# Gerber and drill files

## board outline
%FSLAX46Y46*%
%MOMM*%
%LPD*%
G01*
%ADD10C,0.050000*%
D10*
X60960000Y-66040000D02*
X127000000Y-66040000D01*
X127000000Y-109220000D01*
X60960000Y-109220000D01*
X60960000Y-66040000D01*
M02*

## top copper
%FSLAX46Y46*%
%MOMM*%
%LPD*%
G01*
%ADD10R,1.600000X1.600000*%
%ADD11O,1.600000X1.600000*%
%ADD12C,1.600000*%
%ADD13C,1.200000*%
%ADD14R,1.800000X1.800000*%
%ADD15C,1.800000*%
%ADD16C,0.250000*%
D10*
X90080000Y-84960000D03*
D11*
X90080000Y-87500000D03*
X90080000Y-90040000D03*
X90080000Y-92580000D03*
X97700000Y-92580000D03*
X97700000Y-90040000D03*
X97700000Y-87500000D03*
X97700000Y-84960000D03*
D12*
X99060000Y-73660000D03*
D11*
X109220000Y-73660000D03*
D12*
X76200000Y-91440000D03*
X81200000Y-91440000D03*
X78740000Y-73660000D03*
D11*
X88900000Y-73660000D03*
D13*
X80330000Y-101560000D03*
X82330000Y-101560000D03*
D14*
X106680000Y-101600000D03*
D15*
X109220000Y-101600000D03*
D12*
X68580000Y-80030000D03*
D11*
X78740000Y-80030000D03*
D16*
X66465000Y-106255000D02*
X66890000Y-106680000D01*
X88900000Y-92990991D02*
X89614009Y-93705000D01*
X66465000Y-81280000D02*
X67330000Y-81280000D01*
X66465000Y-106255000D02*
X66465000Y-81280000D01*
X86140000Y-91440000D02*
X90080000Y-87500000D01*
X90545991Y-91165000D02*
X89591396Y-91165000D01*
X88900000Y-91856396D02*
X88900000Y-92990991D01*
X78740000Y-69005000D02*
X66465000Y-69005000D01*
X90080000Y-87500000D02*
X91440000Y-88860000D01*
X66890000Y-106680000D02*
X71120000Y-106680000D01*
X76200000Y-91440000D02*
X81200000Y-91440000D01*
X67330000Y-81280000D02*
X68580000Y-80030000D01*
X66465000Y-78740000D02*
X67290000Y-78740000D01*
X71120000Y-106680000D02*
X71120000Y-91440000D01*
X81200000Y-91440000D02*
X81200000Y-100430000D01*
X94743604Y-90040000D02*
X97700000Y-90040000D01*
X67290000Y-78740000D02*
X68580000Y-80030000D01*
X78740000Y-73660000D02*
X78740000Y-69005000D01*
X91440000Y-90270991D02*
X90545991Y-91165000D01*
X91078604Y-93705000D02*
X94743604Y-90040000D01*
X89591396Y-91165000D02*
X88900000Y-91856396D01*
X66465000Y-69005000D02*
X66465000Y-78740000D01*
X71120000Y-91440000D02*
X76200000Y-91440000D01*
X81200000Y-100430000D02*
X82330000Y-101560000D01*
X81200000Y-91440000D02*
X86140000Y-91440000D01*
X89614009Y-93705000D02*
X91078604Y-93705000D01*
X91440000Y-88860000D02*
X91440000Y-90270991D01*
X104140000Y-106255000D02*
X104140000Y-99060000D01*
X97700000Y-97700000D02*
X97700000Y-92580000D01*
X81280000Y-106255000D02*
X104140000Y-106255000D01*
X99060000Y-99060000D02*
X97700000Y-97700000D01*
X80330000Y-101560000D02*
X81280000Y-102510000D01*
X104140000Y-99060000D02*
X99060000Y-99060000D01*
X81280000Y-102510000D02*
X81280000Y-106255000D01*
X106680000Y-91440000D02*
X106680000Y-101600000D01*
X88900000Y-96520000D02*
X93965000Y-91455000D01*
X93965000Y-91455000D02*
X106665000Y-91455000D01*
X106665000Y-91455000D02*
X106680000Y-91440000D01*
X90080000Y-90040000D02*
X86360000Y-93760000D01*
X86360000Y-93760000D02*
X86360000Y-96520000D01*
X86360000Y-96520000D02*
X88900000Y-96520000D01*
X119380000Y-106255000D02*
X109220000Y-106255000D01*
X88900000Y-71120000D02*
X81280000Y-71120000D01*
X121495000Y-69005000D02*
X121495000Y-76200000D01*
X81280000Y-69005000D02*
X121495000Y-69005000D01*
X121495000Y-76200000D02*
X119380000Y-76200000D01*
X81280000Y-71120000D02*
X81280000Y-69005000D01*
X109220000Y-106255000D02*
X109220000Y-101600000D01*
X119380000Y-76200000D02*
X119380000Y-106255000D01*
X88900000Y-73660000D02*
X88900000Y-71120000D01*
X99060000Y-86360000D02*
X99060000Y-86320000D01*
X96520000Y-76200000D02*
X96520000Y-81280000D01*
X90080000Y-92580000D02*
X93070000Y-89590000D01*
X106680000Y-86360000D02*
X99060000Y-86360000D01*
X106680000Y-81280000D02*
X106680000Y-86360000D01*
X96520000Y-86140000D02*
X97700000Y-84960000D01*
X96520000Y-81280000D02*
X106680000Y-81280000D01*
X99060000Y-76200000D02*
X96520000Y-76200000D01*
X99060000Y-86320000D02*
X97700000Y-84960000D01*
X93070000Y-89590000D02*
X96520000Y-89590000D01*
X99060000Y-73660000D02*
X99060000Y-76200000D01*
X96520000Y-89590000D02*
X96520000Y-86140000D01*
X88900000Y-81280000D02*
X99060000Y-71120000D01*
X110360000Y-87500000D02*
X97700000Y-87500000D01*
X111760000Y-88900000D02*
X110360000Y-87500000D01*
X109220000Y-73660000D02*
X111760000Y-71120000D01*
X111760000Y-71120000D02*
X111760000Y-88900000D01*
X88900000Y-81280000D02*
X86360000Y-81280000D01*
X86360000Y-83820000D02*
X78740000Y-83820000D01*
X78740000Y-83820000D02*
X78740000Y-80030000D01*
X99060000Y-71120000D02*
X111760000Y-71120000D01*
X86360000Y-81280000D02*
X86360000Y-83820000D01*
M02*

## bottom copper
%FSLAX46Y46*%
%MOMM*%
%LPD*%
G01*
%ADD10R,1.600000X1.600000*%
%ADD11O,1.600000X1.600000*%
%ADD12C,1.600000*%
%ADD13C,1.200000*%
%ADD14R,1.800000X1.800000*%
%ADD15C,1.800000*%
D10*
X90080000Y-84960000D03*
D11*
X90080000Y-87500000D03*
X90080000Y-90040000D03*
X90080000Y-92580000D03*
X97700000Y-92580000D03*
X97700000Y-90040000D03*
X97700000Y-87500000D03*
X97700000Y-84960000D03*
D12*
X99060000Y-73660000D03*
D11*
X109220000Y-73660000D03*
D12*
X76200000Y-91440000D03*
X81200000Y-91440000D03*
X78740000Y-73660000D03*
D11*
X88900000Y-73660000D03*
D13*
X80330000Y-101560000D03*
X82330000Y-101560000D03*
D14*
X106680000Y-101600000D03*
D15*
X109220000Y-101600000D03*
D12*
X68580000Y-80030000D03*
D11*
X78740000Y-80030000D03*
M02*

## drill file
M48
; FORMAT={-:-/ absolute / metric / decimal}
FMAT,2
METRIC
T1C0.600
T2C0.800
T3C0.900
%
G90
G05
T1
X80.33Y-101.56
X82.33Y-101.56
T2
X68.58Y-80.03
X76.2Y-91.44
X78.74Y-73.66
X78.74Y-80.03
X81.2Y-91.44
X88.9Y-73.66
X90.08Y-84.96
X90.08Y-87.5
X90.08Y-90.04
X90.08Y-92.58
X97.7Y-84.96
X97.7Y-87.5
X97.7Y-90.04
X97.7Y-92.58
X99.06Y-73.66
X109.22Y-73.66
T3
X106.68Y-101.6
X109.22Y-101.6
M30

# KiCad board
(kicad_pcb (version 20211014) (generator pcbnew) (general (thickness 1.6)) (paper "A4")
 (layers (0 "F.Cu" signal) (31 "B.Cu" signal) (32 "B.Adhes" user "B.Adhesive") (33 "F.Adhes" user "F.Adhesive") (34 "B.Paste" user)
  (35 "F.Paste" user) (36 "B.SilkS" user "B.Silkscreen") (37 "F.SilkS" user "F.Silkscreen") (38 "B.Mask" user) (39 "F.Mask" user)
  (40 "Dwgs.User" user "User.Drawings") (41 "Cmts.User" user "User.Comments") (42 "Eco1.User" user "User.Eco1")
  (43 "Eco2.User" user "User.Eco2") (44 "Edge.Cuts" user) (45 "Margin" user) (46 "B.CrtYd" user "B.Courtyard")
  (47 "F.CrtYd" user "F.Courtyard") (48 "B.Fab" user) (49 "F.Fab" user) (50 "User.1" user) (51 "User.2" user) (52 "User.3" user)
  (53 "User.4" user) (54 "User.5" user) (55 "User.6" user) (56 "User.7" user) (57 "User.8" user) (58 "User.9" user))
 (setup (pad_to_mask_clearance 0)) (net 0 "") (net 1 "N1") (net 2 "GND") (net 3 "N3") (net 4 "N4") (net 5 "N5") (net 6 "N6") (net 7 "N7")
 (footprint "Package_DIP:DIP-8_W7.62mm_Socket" (layer "F.Cu") (at 90.08 84.96)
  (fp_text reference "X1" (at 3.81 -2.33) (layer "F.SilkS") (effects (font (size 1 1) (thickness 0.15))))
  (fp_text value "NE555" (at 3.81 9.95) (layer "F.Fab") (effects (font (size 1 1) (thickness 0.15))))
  (pad "1" thru_hole rect (at 0 0) (size 1.6 1.6) (drill 0.8) (layers *.Cu *.Mask) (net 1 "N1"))
  (pad "2" thru_hole oval (at 0 2.54) (size 1.6 1.6) (drill 0.8) (layers *.Cu *.Mask) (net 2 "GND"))
  (pad "3" thru_hole oval (at 0 5.08) (size 1.6 1.6) (drill 0.8) (layers *.Cu *.Mask) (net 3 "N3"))
  (pad "4" thru_hole oval (at 0 7.62) (size 1.6 1.6) (drill 0.8) (layers *.Cu *.Mask) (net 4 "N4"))
  (pad "5" thru_hole oval (at 7.62 7.62) (size 1.6 1.6) (drill 0.8) (layers *.Cu *.Mask) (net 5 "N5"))
  (pad "6" thru_hole oval (at 7.62 5.08) (size 1.6 1.6) (drill 0.8) (layers *.Cu *.Mask) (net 2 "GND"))
  (pad "7" thru_hole oval (at 7.62 2.54) (size 1.6 1.6) (drill 0.8) (layers *.Cu *.Mask) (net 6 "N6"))
  (pad "8" thru_hole oval (at 7.62 0) (size 1.6 1.6) (drill 0.8) (layers *.Cu *.Mask) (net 4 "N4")))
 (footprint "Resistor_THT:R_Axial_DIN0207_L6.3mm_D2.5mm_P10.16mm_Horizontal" (layer "F.Cu") (at 99.06 73.66)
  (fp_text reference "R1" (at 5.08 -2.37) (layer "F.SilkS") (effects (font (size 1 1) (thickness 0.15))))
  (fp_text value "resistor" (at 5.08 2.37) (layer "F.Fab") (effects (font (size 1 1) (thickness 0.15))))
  (pad "1" thru_hole circle (at 0 0) (size 1.6 1.6) (drill 0.8) (layers *.Cu *.Mask) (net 4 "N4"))
  (pad "2" thru_hole oval (at 10.16 0) (size 1.6 1.6) (drill 0.8) (layers *.Cu *.Mask) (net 6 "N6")))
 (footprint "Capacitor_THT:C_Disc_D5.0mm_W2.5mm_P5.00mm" (layer "F.Cu") (at 76.2 91.44)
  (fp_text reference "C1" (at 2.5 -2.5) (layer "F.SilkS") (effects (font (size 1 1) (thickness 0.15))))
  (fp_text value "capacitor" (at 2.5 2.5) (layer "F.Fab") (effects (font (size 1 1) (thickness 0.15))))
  (pad "1" thru_hole circle (at 0 0) (size 1.6 1.6) (drill 0.8) (layers *.Cu *.Mask) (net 2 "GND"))
  (pad "2" thru_hole circle (at 5 0) (size 1.6 1.6) (drill 0.8) (layers *.Cu *.Mask) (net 2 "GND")))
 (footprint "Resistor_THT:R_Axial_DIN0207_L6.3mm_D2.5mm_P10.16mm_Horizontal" (layer "F.Cu") (at 78.74 73.66)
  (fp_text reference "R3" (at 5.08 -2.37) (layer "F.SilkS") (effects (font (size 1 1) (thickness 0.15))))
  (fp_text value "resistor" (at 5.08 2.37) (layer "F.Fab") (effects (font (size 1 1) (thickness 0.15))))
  (pad "1" thru_hole circle (at 0 0) (size 1.6 1.6) (drill 0.8) (layers *.Cu *.Mask) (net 2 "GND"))
  (pad "2" thru_hole oval (at 10.16 0) (size 1.6 1.6) (drill 0.8) (layers *.Cu *.Mask) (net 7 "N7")))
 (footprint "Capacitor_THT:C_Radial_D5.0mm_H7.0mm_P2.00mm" (layer "F.Cu") (at 80.33 101.56)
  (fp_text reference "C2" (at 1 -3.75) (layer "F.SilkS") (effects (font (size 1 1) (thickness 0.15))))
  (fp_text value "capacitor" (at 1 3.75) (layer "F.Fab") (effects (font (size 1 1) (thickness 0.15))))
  (pad "1" thru_hole circle (at 0 0) (size 1.2 1.2) (drill 0.6) (layers *.Cu *.Mask) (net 5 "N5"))
  (pad "2" thru_hole circle (at 2 0) (size 1.2 1.2) (drill 0.6) (layers *.Cu *.Mask) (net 2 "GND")))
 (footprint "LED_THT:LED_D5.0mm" (layer "F.Cu") (at 106.68 101.6)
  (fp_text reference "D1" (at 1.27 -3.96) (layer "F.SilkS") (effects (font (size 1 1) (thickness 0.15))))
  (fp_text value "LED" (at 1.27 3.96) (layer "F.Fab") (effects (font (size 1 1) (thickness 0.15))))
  (pad "1" thru_hole rect (at 0 0) (size 1.8 1.8) (drill 0.9) (layers *.Cu *.Mask) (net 3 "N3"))
  (pad "2" thru_hole circle (at 2.54 0) (size 1.8 1.8) (drill 0.9) (layers *.Cu *.Mask) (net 7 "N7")))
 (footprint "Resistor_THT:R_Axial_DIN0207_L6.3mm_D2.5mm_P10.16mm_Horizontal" (layer "F.Cu") (at 68.58 80.03)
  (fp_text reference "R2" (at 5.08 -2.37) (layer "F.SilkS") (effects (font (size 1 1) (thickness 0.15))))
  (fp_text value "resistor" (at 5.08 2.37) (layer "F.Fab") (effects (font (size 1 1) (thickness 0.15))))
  (pad "1" thru_hole circle (at 0 0) (size 1.6 1.6) (drill 0.8) (layers *.Cu *.Mask) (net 2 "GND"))
  (pad "2" thru_hole oval (at 10.16 0) (size 1.6 1.6) (drill 0.8) (layers *.Cu *.Mask) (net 6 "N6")))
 (gr_rect (start 127 66.04) (end 60.96 109.22) (layer "Edge.Cuts") (width 0.05) (fill none))
 (segment (start 66.465 106.255) (end 66.89 106.68) (width 0.25) (layer "F.Cu") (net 2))
 (segment (start 88.9 92.990991) (end 89.614009 93.705) (width 0.25) (layer "F.Cu") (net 2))
 (segment (start 66.465 81.28) (end 67.33 81.28) (width 0.25) (layer "F.Cu") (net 2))
 (segment (start 66.465 106.255) (end 66.465 81.28) (width 0.25) (layer "F.Cu") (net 2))
 (segment (start 86.14 91.44) (end 90.08 87.5) (width 0.25) (layer "F.Cu") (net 2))
 (segment (start 90.545991 91.165) (end 89.591396 91.165) (width 0.25) (layer "F.Cu") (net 2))
 (segment (start 88.9 91.856396) (end 88.9 92.990991) (width 0.25) (layer "F.Cu") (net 2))
 (segment (start 78.74 69.005) (end 66.465 69.005) (width 0.25) (layer "F.Cu") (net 2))
 (segment (start 90.08 87.5) (end 91.44 88.86) (width 0.25) (layer "F.Cu") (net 2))
 (segment (start 66.89 106.68) (end 71.12 106.68) (width 0.25) (layer "F.Cu") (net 2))
 (segment (start 76.2 91.44) (end 81.2 91.44) (width 0.25) (layer "F.Cu") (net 2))
 (segment (start 67.33 81.28) (end 68.58 80.03) (width 0.25) (layer "F.Cu") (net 2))
 (segment (start 66.465 78.74) (end 67.29 78.74) (width 0.25) (layer "F.Cu") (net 2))
 (segment (start 71.12 106.68) (end 71.12 91.44) (width 0.25) (layer "F.Cu") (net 2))
 (segment (start 81.2 91.44) (end 81.2 100.43) (width 0.25) (layer "F.Cu") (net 2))
 (segment (start 94.743604 90.04) (end 97.7 90.04) (width 0.25) (layer "F.Cu") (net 2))
 (segment (start 67.29 78.74) (end 68.58 80.03) (width 0.25) (layer "F.Cu") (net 2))
 (segment (start 78.74 73.66) (end 78.74 69.005) (width 0.25) (layer "F.Cu") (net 2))
 (segment (start 91.44 90.270991) (end 90.545991 91.165) (width 0.25) (layer "F.Cu") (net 2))
 (segment (start 91.078604 93.705) (end 94.743604 90.04) (width 0.25) (layer "F.Cu") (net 2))
 (segment (start 89.591396 91.165) (end 88.9 91.856396) (width 0.25) (layer "F.Cu") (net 2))
 (segment (start 66.465 69.005) (end 66.465 78.74) (width 0.25) (layer "F.Cu") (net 2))
 (segment (start 71.12 91.44) (end 76.2 91.44) (width 0.25) (layer "F.Cu") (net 2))
 (segment (start 81.2 100.43) (end 82.33 101.56) (width 0.25) (layer "F.Cu") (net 2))
 (segment (start 81.2 91.44) (end 86.14 91.44) (width 0.25) (layer "F.Cu") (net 2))
 (segment (start 89.614009 93.705) (end 91.078604 93.705) (width 0.25) (layer "F.Cu") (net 2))
 (segment (start 91.44 88.86) (end 91.44 90.270991) (width 0.25) (layer "F.Cu") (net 2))
 (segment (start 104.14 106.255) (end 104.14 99.06) (width 0.25) (layer "F.Cu") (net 5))
 (segment (start 97.7 97.7) (end 97.7 92.58) (width 0.25) (layer "F.Cu") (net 5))
 (segment (start 81.28 106.255) (end 104.14 106.255) (width 0.25) (layer "F.Cu") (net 5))
 (segment (start 99.06 99.06) (end 97.7 97.7) (width 0.25) (layer "F.Cu") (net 5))
 (segment (start 80.33 101.56) (end 81.28 102.51) (width 0.25) (layer "F.Cu") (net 5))
 (segment (start 104.14 99.06) (end 99.06 99.06) (width 0.25) (layer "F.Cu") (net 5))
 (segment (start 81.28 102.51) (end 81.28 106.255) (width 0.25) (layer "F.Cu") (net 5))
 (segment (start 106.68 91.44) (end 106.68 101.6) (width 0.25) (layer "F.Cu") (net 3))
 (segment (start 88.9 96.52) (end 93.965 91.455) (width 0.25) (layer "F.Cu") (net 3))
 (segment (start 93.965 91.455) (end 106.665 91.455) (width 0.25) (layer "F.Cu") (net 3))
 (segment (start 106.665 91.455) (end 106.68 91.44) (width 0.25) (layer "F.Cu") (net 3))
 (segment (start 90.08 90.04) (end 86.36 93.76) (width 0.25) (layer "F.Cu") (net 3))
 (segment (start 86.36 93.76) (end 86.36 96.52) (width 0.25) (layer "F.Cu") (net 3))
 (segment (start 86.36 96.52) (end 88.9 96.52) (width 0.25) (layer "F.Cu") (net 3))
 (segment (start 119.38 106.255) (end 109.22 106.255) (width 0.25) (layer "F.Cu") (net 7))
 (segment (start 88.9 71.12) (end 81.28 71.12) (width 0.25) (layer "F.Cu") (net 7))
 (segment (start 121.495 69.005) (end 121.495 76.2) (width 0.25) (layer "F.Cu") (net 7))
 (segment (start 81.28 69.005) (end 121.495 69.005) (width 0.25) (layer "F.Cu") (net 7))
 (segment (start 121.495 76.2) (end 119.38 76.2) (width 0.25) (layer "F.Cu") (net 7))
 (segment (start 81.28 71.12) (end 81.28 69.005) (width 0.25) (layer "F.Cu") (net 7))
 (segment (start 109.22 106.255) (end 109.22 101.6) (width 0.25) (layer "F.Cu") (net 7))
 (segment (start 119.38 76.2) (end 119.38 106.255) (width 0.25) (layer "F.Cu") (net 7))
 (segment (start 88.9 73.66) (end 88.9 71.12) (width 0.25) (layer "F.Cu") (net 7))
 (segment (start 99.06 86.36) (end 99.06 86.32) (width 0.25) (layer "F.Cu") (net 4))
 (segment (start 96.52 76.2) (end 96.52 81.28) (width 0.25) (layer "F.Cu") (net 4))
 (segment (start 90.08 92.58) (end 93.07 89.59) (width 0.25) (layer "F.Cu") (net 4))
 (segment (start 106.68 86.36) (end 99.06 86.36) (width 0.25) (layer "F.Cu") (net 4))
 (segment (start 106.68 81.28) (end 106.68 86.36) (width 0.25) (layer "F.Cu") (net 4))
 (segment (start 96.52 86.14) (end 97.7 84.96) (width 0.25) (layer "F.Cu") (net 4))
 (segment (start 96.52 81.28) (end 106.68 81.28) (width 0.25) (layer "F.Cu") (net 4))
 (segment (start 99.06 76.2) (end 96.52 76.2) (width 0.25) (layer "F.Cu") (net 4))
 (segment (start 99.06 86.32) (end 97.7 84.96) (width 0.25) (layer "F.Cu") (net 4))
 (segment (start 93.07 89.59) (end 96.52 89.59) (width 0.25) (layer "F.Cu") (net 4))
 (segment (start 99.06 73.66) (end 99.06 76.2) (width 0.25) (layer "F.Cu") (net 4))
 (segment (start 96.52 89.59) (end 96.52 86.14) (width 0.25) (layer "F.Cu") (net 4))
 (segment (start 88.9 81.28) (end 99.06 71.12) (width 0.25) (layer "F.Cu") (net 6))
 (segment (start 110.36 87.5) (end 97.7 87.5) (width 0.25) (layer "F.Cu") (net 6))
 (segment (start 111.76 88.9) (end 110.36 87.5) (width 0.25) (layer "F.Cu") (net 6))
 (segment (start 109.22 73.66) (end 111.76 71.12) (width 0.25) (layer "F.Cu") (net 6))
 (segment (start 111.76 71.12) (end 111.76 88.9) (width 0.25) (layer "F.Cu") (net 6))
 (segment (start 88.9 81.28) (end 86.36 81.28) (width 0.25) (layer "F.Cu") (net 6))
 (segment (start 86.36 83.82) (end 78.74 83.82) (width 0.25) (layer "F.Cu") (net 6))
 (segment (start 78.74 83.82) (end 78.74 80.03) (width 0.25) (layer "F.Cu") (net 6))
 (segment (start 99.06 71.12) (end 111.76 71.12) (width 0.25) (layer "F.Cu") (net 6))
 (segment (start 86.36 81.28) (end 86.36 83.82) (width 0.25) (layer "F.Cu") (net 6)))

